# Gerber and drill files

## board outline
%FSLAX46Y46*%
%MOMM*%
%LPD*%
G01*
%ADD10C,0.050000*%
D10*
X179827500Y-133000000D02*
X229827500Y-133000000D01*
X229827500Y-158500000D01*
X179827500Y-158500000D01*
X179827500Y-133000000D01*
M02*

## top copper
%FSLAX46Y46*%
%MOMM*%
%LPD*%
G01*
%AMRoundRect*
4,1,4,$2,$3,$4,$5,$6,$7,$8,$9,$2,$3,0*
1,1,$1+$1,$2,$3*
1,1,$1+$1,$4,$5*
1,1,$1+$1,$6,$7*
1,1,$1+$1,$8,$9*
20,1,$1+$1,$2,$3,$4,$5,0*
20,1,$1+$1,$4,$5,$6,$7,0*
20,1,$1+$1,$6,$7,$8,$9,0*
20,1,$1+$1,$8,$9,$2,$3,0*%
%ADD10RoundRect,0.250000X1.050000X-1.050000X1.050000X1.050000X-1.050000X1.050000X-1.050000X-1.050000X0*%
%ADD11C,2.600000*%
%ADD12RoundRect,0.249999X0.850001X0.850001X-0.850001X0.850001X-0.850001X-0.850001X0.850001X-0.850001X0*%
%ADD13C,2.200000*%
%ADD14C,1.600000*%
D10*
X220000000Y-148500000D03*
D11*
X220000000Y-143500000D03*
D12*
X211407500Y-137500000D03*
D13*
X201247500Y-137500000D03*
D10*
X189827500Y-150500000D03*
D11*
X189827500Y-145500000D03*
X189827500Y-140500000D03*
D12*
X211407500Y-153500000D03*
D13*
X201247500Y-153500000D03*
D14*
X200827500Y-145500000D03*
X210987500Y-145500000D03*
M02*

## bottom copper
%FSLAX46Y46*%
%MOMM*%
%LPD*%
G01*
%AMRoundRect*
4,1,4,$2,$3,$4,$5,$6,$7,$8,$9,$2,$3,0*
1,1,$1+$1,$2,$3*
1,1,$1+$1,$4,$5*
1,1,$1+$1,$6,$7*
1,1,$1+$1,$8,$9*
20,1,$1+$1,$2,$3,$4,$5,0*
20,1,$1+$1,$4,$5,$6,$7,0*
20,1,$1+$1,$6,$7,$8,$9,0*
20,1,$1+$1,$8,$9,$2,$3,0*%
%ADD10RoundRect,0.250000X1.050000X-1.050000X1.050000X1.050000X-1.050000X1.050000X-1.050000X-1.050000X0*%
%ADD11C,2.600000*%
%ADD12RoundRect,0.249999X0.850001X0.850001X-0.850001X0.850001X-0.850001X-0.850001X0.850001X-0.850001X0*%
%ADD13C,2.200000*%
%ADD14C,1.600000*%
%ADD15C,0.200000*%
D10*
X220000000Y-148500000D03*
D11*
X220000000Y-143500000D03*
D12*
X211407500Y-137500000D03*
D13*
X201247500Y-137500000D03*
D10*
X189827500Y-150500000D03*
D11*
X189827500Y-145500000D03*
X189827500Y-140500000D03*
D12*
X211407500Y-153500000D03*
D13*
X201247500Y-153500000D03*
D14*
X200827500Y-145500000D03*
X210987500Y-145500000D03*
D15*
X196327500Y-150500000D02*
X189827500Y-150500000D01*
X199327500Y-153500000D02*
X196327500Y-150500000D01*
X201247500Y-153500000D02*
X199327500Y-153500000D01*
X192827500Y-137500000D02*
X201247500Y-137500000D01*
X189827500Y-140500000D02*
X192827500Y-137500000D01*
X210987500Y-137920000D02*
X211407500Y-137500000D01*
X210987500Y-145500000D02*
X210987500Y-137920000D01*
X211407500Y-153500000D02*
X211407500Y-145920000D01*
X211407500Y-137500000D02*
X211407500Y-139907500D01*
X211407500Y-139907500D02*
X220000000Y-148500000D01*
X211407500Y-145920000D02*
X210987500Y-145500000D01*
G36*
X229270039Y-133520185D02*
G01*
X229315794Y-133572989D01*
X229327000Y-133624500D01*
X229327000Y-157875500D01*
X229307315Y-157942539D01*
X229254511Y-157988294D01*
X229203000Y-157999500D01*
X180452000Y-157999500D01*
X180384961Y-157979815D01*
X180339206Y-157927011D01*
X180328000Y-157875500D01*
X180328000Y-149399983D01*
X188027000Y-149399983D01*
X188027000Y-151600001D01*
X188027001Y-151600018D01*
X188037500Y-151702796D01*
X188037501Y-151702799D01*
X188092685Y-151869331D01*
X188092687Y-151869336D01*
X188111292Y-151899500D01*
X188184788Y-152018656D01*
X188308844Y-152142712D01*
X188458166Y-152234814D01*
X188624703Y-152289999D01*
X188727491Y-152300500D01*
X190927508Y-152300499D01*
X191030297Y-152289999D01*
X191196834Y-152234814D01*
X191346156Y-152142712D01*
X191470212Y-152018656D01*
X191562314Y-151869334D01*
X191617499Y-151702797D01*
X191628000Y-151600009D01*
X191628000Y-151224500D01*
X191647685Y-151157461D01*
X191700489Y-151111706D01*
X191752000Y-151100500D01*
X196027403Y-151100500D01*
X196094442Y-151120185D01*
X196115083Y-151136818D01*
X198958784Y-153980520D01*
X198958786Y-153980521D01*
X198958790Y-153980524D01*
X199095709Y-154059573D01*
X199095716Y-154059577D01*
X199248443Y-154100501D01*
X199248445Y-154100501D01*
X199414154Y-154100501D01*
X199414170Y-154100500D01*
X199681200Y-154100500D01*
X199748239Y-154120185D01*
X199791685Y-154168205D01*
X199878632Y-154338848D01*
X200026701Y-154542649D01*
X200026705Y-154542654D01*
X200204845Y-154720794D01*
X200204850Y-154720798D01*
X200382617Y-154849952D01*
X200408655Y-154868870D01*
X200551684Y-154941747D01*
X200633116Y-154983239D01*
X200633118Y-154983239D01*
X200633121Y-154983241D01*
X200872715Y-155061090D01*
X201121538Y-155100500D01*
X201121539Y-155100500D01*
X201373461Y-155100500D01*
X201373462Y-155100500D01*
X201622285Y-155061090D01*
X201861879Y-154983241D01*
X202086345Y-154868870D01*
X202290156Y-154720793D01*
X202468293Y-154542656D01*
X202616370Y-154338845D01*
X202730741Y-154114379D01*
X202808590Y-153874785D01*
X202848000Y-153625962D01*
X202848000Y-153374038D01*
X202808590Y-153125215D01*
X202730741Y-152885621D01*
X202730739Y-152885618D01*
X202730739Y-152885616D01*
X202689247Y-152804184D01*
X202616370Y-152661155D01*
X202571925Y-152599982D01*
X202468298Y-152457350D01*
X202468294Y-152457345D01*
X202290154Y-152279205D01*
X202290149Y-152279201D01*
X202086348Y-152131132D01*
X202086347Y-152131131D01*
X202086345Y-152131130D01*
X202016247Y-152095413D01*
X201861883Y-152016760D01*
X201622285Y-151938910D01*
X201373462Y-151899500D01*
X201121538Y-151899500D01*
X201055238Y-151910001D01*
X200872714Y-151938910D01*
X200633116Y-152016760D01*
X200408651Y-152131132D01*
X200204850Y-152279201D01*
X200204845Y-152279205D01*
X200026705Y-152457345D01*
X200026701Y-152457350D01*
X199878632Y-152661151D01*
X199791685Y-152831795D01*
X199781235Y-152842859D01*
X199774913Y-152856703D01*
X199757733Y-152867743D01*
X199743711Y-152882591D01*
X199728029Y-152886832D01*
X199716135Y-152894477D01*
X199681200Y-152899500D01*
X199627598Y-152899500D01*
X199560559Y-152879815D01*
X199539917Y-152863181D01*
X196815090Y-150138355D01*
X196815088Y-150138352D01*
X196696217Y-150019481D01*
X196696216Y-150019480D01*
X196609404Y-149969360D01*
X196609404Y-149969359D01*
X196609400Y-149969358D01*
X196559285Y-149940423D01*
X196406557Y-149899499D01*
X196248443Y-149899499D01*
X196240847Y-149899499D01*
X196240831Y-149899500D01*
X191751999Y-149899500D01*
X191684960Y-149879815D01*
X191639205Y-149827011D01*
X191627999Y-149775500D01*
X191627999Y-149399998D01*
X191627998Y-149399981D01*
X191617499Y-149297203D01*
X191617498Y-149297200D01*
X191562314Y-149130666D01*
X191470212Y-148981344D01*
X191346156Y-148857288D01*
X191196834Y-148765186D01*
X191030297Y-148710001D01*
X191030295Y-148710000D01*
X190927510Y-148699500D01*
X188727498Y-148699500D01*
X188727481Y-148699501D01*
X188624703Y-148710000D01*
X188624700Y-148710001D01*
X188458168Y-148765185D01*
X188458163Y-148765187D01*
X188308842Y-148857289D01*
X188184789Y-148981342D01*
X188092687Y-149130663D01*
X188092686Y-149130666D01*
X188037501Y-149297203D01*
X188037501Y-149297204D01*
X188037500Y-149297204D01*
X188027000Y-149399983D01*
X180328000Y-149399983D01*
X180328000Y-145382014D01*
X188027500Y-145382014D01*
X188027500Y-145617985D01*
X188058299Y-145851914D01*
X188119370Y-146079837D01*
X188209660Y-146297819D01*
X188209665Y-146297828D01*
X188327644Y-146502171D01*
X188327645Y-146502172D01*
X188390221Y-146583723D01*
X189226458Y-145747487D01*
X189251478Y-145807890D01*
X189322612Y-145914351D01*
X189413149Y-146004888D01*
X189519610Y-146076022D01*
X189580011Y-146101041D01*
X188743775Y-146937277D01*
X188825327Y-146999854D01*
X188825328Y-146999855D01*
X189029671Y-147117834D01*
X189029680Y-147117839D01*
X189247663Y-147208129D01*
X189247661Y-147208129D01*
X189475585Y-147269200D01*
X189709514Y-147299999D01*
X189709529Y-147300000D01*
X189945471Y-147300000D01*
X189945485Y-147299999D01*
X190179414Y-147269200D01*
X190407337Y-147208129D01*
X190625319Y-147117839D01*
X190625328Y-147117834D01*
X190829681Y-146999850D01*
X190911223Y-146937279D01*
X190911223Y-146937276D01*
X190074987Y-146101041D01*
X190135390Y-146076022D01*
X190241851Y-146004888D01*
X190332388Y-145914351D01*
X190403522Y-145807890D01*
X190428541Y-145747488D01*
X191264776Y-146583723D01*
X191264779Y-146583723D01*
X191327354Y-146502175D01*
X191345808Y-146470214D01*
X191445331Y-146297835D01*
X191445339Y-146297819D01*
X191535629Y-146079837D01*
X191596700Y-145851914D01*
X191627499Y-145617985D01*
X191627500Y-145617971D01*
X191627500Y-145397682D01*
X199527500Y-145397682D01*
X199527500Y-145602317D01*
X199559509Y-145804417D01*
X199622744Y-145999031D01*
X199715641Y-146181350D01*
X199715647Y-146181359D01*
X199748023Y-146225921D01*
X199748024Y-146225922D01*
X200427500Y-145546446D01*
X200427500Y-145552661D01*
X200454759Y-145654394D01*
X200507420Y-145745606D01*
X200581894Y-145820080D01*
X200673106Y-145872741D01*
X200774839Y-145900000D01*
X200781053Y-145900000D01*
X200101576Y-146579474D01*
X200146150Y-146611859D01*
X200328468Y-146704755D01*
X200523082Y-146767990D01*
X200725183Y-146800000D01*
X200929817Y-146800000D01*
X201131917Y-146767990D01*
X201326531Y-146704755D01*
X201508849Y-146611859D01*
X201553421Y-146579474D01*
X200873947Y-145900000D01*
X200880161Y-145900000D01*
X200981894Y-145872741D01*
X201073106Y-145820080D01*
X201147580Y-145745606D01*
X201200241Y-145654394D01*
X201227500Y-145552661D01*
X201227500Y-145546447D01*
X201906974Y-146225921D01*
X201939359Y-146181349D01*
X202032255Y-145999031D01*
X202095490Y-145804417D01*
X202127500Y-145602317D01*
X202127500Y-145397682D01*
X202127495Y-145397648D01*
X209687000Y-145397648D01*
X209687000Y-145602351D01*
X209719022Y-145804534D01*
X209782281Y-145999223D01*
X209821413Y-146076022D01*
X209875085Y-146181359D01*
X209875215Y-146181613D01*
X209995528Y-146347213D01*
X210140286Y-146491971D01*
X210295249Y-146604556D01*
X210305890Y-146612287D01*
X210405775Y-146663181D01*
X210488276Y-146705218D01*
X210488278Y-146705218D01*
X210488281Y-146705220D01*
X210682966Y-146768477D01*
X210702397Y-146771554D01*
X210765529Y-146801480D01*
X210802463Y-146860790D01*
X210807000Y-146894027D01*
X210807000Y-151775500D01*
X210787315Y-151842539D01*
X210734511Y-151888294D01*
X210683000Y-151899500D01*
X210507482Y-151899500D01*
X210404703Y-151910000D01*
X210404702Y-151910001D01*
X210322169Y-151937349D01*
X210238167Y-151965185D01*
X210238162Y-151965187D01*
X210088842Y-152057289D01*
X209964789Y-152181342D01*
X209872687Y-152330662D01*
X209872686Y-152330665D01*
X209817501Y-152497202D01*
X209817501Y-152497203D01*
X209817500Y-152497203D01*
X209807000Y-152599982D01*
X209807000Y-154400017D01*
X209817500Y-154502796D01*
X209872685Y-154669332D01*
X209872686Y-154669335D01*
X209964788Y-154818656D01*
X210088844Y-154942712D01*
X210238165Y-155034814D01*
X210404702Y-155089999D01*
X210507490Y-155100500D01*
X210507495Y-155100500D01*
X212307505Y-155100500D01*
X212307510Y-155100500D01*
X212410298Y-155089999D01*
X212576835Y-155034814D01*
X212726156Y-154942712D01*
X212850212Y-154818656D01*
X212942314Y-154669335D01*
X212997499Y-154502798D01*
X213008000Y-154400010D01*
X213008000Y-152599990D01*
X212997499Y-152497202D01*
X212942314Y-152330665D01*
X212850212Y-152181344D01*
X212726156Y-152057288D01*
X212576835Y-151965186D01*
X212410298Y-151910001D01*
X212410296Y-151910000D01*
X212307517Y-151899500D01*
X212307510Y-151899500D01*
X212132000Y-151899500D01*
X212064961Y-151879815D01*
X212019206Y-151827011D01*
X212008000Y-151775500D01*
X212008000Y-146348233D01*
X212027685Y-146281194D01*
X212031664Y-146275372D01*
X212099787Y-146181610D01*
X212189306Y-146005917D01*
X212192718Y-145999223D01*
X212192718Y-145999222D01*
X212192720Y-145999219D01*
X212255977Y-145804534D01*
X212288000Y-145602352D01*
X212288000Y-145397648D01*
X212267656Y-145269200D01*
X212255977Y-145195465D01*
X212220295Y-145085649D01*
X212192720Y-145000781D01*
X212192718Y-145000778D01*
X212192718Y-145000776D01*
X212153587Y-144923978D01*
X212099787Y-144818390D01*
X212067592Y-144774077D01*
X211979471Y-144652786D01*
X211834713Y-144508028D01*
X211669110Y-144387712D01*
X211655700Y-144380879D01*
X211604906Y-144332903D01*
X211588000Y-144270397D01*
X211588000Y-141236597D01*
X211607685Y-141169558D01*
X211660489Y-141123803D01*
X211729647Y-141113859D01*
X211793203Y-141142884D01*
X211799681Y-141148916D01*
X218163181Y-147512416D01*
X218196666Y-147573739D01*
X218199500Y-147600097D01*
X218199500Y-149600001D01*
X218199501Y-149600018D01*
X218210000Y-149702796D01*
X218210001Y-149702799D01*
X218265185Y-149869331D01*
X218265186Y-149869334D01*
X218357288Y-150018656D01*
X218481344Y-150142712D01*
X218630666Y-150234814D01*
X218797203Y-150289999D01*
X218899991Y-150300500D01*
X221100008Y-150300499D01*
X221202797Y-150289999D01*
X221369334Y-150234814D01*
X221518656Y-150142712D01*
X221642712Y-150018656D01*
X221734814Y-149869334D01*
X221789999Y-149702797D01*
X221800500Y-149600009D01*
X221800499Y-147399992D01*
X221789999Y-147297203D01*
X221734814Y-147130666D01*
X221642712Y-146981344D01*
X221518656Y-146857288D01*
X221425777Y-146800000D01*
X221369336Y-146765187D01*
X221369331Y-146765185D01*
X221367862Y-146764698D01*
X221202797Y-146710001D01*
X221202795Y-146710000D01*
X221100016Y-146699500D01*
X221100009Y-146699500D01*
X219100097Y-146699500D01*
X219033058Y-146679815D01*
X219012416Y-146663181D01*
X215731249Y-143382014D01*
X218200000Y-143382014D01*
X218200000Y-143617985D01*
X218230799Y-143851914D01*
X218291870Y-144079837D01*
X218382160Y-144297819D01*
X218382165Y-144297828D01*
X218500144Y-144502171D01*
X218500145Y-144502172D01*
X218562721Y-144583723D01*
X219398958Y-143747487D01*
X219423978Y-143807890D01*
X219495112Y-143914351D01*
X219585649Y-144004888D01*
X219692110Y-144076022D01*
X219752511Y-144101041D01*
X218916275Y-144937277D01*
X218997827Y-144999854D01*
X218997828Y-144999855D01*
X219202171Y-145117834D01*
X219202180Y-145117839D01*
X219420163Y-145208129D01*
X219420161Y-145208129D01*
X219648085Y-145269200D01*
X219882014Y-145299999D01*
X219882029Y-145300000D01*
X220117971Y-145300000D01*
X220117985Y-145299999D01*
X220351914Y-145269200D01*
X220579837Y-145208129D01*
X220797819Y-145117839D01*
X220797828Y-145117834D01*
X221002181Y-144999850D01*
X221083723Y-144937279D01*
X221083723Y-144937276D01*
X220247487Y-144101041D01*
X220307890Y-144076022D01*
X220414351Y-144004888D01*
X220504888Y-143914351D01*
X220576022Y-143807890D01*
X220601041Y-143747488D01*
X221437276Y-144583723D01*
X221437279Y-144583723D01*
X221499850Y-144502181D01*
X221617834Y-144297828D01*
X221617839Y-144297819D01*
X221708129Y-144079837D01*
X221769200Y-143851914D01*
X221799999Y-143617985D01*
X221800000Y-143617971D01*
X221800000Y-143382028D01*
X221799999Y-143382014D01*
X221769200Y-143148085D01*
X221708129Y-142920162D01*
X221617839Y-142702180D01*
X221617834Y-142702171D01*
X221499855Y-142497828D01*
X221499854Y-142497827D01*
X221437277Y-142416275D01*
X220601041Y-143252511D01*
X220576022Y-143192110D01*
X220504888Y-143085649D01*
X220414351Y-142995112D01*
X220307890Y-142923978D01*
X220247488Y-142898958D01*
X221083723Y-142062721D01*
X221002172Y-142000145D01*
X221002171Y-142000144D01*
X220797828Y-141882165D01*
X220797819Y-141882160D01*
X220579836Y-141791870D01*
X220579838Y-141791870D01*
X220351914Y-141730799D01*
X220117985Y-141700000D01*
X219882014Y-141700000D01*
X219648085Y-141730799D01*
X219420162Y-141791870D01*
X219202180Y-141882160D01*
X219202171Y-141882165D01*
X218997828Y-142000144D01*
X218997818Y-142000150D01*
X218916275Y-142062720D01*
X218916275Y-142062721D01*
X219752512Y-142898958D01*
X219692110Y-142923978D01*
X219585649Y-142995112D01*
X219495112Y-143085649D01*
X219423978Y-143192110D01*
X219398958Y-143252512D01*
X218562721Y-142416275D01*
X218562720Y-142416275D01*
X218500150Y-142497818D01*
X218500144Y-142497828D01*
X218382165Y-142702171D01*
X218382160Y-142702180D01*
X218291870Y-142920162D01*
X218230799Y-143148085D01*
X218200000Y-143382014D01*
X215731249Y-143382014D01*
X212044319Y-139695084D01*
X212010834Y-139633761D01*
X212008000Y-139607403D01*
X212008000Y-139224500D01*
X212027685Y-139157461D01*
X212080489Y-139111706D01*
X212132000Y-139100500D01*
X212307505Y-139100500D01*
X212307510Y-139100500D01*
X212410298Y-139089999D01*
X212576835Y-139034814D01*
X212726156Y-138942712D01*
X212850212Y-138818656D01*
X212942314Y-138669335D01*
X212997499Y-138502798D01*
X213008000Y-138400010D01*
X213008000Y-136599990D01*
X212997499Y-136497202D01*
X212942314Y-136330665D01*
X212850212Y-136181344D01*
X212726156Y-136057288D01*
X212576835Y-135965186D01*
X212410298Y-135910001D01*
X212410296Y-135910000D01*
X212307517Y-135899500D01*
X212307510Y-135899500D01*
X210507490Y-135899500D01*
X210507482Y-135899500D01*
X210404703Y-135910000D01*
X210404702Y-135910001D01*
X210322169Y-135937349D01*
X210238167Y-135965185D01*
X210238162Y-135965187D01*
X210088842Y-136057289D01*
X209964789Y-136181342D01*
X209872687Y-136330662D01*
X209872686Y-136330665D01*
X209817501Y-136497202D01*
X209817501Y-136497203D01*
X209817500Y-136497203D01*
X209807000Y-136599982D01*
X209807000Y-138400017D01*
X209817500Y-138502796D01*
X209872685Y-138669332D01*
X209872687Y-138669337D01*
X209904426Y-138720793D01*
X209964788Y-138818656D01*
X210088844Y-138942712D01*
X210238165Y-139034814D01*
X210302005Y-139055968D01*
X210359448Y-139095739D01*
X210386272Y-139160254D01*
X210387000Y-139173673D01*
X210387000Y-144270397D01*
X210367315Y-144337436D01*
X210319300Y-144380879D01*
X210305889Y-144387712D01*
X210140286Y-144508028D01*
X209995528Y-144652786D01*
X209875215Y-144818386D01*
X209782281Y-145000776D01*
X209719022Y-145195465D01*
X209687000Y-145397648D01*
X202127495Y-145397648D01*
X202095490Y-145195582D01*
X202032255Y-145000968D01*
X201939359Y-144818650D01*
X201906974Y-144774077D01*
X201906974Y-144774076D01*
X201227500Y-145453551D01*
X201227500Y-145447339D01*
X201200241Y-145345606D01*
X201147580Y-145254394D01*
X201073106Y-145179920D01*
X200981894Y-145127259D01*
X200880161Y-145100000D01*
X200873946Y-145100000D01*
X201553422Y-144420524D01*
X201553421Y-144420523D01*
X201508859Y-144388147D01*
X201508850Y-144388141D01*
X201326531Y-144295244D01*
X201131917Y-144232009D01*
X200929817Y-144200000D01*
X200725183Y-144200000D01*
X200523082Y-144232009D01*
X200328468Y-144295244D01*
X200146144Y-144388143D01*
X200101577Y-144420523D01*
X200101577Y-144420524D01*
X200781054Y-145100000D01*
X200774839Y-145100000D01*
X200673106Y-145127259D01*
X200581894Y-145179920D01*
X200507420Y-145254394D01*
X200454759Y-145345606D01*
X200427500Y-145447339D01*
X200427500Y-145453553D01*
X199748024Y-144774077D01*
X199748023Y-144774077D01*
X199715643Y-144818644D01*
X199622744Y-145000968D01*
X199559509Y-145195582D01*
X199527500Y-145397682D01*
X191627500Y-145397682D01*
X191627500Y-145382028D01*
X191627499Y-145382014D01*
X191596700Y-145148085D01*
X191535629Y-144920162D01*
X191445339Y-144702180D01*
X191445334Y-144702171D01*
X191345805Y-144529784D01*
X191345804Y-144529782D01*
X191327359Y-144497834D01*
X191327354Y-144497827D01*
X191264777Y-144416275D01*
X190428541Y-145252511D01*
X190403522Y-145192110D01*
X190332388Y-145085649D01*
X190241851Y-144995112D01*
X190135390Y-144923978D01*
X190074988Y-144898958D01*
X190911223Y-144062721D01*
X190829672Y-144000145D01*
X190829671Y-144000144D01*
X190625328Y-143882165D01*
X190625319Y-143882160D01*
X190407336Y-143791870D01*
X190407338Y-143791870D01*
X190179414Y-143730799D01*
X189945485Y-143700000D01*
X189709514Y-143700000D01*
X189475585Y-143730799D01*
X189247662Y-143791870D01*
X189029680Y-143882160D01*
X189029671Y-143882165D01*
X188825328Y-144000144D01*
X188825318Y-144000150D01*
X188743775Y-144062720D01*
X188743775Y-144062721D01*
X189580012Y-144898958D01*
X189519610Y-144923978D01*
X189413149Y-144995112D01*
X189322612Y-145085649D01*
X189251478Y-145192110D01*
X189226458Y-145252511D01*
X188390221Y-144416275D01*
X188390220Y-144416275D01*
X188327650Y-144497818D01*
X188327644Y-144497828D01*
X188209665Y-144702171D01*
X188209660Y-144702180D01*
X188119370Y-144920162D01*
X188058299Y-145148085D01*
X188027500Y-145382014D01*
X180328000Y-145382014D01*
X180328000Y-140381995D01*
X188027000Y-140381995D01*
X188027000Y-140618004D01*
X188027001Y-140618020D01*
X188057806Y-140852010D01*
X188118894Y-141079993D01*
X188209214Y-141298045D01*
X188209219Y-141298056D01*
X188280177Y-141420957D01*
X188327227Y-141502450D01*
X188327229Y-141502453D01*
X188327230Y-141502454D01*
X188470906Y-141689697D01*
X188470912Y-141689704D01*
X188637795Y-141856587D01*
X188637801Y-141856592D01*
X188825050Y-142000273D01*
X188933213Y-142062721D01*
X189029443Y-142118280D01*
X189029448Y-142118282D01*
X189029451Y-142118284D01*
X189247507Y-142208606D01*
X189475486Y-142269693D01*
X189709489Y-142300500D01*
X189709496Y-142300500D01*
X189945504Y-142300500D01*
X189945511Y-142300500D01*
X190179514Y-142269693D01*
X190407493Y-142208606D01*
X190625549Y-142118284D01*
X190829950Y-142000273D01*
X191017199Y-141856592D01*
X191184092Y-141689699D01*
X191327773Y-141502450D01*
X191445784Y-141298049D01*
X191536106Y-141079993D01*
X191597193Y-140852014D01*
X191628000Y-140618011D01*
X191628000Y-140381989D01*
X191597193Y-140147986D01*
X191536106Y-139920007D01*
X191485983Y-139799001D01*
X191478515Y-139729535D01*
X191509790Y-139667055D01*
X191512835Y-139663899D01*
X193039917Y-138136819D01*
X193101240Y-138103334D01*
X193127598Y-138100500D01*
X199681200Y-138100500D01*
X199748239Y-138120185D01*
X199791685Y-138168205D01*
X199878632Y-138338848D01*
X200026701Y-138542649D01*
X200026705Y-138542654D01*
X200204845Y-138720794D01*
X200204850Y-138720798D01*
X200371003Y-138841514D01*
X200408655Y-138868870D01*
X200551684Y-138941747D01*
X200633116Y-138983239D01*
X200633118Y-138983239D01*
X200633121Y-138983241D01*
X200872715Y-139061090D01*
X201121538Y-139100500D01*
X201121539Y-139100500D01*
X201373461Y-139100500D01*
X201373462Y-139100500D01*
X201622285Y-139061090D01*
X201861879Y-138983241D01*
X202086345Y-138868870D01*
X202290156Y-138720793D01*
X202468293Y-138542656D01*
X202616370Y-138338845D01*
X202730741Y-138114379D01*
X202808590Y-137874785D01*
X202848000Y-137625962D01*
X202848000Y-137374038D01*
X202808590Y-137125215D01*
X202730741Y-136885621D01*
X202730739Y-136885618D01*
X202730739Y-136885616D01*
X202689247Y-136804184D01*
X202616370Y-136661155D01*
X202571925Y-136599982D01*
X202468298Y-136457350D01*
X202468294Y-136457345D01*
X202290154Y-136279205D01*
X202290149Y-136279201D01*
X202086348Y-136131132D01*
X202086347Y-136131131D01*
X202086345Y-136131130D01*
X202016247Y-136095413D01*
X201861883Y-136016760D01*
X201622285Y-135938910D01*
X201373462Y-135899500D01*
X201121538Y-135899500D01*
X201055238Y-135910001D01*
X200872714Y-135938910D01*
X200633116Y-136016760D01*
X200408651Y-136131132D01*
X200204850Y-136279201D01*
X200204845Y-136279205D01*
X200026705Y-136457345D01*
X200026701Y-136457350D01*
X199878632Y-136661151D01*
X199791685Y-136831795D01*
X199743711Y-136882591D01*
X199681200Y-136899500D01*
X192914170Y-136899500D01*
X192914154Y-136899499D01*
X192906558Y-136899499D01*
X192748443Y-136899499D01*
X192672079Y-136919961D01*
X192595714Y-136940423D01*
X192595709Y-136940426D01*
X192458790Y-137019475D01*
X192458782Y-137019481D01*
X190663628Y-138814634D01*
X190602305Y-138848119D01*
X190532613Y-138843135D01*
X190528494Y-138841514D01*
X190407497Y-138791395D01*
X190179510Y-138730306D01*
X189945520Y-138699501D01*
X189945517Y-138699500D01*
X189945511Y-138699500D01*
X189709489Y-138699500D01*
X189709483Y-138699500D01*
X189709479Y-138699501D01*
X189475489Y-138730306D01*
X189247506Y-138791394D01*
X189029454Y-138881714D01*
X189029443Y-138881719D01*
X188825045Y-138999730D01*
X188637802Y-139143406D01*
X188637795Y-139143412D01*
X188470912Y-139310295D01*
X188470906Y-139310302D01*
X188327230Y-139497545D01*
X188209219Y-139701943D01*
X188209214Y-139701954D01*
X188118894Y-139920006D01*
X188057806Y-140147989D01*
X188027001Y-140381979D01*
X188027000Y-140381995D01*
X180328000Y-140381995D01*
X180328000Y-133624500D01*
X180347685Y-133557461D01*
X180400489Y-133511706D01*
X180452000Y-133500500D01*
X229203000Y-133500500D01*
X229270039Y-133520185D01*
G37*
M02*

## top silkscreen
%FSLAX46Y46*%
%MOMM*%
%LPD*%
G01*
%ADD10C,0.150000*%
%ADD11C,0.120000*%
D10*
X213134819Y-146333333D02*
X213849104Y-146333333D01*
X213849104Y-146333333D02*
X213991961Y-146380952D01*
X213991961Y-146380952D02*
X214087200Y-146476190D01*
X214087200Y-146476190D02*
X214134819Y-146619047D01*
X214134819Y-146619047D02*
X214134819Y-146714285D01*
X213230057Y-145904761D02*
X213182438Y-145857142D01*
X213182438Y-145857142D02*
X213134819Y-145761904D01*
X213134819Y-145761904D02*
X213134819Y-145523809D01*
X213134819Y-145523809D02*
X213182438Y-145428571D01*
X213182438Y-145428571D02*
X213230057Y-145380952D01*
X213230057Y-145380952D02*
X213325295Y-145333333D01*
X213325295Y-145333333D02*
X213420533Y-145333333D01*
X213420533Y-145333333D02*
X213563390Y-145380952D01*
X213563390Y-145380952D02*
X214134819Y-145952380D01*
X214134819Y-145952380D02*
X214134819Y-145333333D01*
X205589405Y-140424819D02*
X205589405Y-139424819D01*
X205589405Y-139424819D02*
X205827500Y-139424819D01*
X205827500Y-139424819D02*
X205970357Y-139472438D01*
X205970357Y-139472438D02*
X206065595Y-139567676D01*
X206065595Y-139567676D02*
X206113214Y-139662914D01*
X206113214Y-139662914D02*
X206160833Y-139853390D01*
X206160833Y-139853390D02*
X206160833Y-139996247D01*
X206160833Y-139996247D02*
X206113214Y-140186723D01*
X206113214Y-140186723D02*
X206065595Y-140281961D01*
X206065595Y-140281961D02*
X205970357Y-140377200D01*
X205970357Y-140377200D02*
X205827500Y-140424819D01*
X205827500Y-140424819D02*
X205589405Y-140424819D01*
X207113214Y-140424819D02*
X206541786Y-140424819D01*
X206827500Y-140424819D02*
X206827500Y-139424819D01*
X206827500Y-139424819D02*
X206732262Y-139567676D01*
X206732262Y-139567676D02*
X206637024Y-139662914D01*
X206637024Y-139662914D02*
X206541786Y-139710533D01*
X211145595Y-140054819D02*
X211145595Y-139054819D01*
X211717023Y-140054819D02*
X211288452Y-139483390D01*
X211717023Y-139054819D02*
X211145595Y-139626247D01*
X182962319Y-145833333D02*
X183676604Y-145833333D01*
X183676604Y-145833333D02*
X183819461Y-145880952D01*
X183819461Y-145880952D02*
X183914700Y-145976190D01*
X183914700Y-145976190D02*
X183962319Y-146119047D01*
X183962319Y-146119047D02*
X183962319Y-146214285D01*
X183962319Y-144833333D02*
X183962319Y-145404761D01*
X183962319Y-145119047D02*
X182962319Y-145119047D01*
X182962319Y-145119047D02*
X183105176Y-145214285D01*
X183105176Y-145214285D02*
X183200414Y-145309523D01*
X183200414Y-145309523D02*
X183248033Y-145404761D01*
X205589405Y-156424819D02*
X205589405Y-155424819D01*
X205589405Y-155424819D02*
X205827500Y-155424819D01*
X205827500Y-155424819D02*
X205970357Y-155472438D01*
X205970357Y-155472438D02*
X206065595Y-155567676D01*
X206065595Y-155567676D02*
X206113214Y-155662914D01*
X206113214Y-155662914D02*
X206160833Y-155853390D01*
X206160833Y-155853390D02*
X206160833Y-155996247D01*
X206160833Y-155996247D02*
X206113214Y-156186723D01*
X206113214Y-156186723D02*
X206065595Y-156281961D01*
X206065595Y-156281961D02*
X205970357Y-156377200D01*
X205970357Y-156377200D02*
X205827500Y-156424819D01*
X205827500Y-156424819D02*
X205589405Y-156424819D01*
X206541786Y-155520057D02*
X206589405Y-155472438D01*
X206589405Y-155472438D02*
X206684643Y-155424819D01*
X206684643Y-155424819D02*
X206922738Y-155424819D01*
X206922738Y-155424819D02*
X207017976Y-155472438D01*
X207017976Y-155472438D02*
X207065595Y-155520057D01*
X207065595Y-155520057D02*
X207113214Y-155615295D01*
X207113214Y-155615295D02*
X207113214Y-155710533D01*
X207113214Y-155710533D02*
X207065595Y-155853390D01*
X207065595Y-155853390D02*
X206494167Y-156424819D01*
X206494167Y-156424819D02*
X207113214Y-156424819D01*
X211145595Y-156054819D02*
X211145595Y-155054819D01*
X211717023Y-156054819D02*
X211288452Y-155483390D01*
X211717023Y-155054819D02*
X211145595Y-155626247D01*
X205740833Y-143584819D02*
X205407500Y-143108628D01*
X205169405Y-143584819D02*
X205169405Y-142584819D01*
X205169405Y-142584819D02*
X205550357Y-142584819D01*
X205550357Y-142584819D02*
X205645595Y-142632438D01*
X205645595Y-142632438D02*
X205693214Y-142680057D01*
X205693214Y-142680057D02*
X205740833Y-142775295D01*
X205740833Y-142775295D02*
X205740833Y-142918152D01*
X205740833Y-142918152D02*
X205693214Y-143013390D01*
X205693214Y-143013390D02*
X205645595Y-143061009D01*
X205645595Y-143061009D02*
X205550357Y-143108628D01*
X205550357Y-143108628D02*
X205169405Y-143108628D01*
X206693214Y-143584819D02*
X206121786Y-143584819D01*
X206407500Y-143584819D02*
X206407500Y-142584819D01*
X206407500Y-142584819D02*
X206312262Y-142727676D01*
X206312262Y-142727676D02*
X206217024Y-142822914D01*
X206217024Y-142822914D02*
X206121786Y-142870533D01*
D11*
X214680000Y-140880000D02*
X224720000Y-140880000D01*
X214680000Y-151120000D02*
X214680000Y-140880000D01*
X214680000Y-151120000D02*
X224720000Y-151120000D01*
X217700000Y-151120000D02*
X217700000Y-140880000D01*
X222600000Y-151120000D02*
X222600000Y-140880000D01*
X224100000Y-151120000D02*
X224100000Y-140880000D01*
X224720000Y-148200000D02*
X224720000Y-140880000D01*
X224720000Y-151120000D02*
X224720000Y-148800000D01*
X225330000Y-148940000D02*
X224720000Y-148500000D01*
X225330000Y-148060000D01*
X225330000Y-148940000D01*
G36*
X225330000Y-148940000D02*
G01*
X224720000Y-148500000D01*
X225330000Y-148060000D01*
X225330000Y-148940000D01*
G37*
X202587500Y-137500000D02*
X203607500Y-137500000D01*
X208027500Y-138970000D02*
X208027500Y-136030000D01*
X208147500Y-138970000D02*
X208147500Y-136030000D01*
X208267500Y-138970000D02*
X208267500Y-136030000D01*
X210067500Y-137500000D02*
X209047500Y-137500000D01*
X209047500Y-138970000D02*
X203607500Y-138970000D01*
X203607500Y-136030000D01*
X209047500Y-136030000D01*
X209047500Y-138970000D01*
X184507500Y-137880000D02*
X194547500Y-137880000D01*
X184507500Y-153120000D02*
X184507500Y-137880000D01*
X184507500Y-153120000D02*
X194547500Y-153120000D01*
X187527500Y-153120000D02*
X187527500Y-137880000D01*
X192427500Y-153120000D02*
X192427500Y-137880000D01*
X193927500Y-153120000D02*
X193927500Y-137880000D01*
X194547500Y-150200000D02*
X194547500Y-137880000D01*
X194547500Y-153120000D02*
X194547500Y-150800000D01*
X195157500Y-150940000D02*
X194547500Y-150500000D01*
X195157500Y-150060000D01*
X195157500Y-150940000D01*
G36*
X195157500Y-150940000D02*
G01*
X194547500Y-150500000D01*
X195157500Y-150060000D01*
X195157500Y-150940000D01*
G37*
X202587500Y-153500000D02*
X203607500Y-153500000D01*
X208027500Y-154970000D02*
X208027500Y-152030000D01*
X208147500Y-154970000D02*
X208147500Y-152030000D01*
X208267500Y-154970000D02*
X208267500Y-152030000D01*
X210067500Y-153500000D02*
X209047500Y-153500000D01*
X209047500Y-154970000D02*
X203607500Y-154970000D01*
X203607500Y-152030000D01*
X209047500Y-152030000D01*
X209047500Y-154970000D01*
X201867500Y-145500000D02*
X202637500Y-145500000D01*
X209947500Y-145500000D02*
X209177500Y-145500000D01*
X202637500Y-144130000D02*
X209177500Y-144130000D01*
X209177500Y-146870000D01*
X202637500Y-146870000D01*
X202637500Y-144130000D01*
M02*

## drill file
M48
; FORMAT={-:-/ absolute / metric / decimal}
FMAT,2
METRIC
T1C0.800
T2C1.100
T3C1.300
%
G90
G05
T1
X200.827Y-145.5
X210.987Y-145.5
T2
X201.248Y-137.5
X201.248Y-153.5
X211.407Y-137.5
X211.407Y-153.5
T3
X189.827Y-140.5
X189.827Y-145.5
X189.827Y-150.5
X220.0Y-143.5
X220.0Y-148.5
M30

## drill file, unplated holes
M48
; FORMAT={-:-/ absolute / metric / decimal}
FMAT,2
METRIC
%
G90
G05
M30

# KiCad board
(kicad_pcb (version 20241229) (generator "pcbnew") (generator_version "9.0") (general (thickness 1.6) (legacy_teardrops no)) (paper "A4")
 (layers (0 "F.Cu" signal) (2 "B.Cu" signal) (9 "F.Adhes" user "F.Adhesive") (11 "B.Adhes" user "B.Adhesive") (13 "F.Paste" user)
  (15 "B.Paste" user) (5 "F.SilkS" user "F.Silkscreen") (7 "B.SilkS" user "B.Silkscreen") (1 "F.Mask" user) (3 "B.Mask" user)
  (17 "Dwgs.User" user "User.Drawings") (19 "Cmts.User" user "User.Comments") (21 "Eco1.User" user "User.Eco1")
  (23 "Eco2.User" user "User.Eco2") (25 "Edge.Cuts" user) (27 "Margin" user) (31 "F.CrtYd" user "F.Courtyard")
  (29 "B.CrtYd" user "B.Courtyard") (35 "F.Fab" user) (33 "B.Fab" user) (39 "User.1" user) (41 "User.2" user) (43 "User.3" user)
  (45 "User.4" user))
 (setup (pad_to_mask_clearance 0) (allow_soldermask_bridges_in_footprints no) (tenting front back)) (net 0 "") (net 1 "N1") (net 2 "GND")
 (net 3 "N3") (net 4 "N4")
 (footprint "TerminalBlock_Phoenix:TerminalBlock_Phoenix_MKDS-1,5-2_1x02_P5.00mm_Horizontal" (layer "F.Cu") (at 220 148.5 90)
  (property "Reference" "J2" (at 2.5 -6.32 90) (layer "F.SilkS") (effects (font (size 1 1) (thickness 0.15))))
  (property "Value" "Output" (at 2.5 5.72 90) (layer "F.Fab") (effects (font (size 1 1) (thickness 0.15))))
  (fp_line (start 7.62 -5.32) (end 7.62 4.72) (stroke (width 0.12) (type solid)) (layer "F.SilkS"))
  (fp_line (start -2.62 -5.32) (end 7.62 -5.32) (stroke (width 0.12) (type solid)) (layer "F.SilkS"))
  (fp_line (start -2.62 -5.32) (end -2.62 4.72) (stroke (width 0.12) (type solid)) (layer "F.SilkS"))
  (fp_line (start -2.62 -2.3) (end 7.62 -2.3) (stroke (width 0.12) (type solid)) (layer "F.SilkS"))
  (fp_line (start -2.62 2.6) (end 7.62 2.6) (stroke (width 0.12) (type solid)) (layer "F.SilkS"))
  (fp_line (start -2.62 4.1) (end 7.62 4.1) (stroke (width 0.12) (type solid)) (layer "F.SilkS"))
  (fp_line (start 0.3 4.72) (end 7.62 4.72) (stroke (width 0.12) (type solid)) (layer "F.SilkS"))
  (fp_line (start -2.62 4.72) (end -0.3 4.72) (stroke (width 0.12) (type solid)) (layer "F.SilkS"))
  (fp_poly (pts (xy 0 4.72) (xy 0.44 5.33) (xy -0.44 5.33)) (stroke (width 0.12) (type solid)) (fill yes) (layer "F.SilkS"))
  (pad "1" thru_hole roundrect (at 0 0 90) (size 2.6 2.6) (drill 1.3) (layers "*.Cu" "*.Mask") (remove_unused_layers no)
   (roundrect_rratio 0.096154) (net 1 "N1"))
  (pad "2" thru_hole circle (at 5 0 90) (size 2.6 2.6) (drill 1.3) (layers "*.Cu" "*.Mask") (remove_unused_layers no) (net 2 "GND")))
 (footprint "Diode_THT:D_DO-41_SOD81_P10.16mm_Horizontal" (layer "F.Cu") (at 211.4075 137.5 180)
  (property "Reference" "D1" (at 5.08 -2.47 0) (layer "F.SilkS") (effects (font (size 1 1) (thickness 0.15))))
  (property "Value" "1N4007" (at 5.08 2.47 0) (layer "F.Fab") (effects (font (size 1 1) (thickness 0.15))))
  (fp_line (start 8.82 0) (end 7.8 0) (stroke (width 0.12) (type solid)) (layer "F.SilkS"))
  (fp_line (start 3.38 -1.47) (end 3.38 1.47) (stroke (width 0.12) (type solid)) (layer "F.SilkS"))
  (fp_line (start 3.26 -1.47) (end 3.26 1.47) (stroke (width 0.12) (type solid)) (layer "F.SilkS"))
  (fp_line (start 3.14 -1.47) (end 3.14 1.47) (stroke (width 0.12) (type solid)) (layer "F.SilkS"))
  (fp_line (start 1.34 0) (end 2.36 0) (stroke (width 0.12) (type solid)) (layer "F.SilkS"))
  (fp_rect (start 2.36 -1.47) (end 7.8 1.47) (stroke (width 0.12) (type solid)) (fill no) (layer "F.SilkS"))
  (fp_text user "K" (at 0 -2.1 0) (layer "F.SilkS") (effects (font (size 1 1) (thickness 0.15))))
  (pad "1" thru_hole roundrect (at 0 0 180) (size 2.2 2.2) (drill 1.1) (layers "*.Cu" "*.Mask") (remove_unused_layers no)
   (roundrect_rratio 0.113636) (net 1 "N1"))
  (pad "2" thru_hole circle (at 10.16 0 180) (size 2.2 2.2) (drill 1.1) (layers "*.Cu" "*.Mask") (remove_unused_layers no) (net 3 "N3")))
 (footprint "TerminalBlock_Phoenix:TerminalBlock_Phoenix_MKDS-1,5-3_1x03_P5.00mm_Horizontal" (layer "F.Cu") (at 189.8275 150.5 90)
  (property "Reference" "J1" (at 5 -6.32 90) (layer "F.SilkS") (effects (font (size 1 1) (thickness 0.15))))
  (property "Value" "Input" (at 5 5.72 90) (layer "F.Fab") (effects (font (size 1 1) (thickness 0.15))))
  (fp_line (start 12.62 -5.32) (end 12.62 4.72) (stroke (width 0.12) (type solid)) (layer "F.SilkS"))
  (fp_line (start -2.62 -5.32) (end 12.62 -5.32) (stroke (width 0.12) (type solid)) (layer "F.SilkS"))
  (fp_line (start -2.62 -5.32) (end -2.62 4.72) (stroke (width 0.12) (type solid)) (layer "F.SilkS"))
  (fp_line (start -2.62 -2.3) (end 12.62 -2.3) (stroke (width 0.12) (type solid)) (layer "F.SilkS"))
  (fp_line (start -2.62 2.6) (end 12.62 2.6) (stroke (width 0.12) (type solid)) (layer "F.SilkS"))
  (fp_line (start -2.62 4.1) (end 12.62 4.1) (stroke (width 0.12) (type solid)) (layer "F.SilkS"))
  (fp_line (start 0.3 4.72) (end 12.62 4.72) (stroke (width 0.12) (type solid)) (layer "F.SilkS"))
  (fp_line (start -2.62 4.72) (end -0.3 4.72) (stroke (width 0.12) (type solid)) (layer "F.SilkS"))
  (fp_poly (pts (xy 0 4.72) (xy 0.44 5.33) (xy -0.44 5.33)) (stroke (width 0.12) (type solid)) (fill yes) (layer "F.SilkS"))
  (pad "1" thru_hole roundrect (at 0 0 90) (size 2.6 2.6) (drill 1.3) (layers "*.Cu" "*.Mask") (remove_unused_layers no)
   (roundrect_rratio 0.096154) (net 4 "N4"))
  (pad "2" thru_hole circle (at 5 0 90) (size 2.6 2.6) (drill 1.3) (layers "*.Cu" "*.Mask") (remove_unused_layers no) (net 2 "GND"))
  (pad "3" thru_hole circle (at 10 0 90) (size 2.6 2.6) (drill 1.3) (layers "*.Cu" "*.Mask") (remove_unused_layers no) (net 3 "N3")))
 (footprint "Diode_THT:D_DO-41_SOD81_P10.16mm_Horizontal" (layer "F.Cu") (at 211.4075 153.5 180)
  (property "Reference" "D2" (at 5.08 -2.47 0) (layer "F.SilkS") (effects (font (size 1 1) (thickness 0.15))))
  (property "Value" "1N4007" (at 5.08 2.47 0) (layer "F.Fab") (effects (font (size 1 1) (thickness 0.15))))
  (fp_line (start 8.82 0) (end 7.8 0) (stroke (width 0.12) (type solid)) (layer "F.SilkS"))
  (fp_line (start 3.38 -1.47) (end 3.38 1.47) (stroke (width 0.12) (type solid)) (layer "F.SilkS"))
  (fp_line (start 3.26 -1.47) (end 3.26 1.47) (stroke (width 0.12) (type solid)) (layer "F.SilkS"))
  (fp_line (start 3.14 -1.47) (end 3.14 1.47) (stroke (width 0.12) (type solid)) (layer "F.SilkS"))
  (fp_line (start 1.34 0) (end 2.36 0) (stroke (width 0.12) (type solid)) (layer "F.SilkS"))
  (fp_rect (start 2.36 -1.47) (end 7.8 1.47) (stroke (width 0.12) (type solid)) (fill no) (layer "F.SilkS"))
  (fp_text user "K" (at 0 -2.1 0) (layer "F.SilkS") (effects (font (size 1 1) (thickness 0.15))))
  (pad "1" thru_hole roundrect (at 0 0 180) (size 2.2 2.2) (drill 1.1) (layers "*.Cu" "*.Mask") (remove_unused_layers no)
   (roundrect_rratio 0.113636) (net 1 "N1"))
  (pad "2" thru_hole circle (at 10.16 0 180) (size 2.2 2.2) (drill 1.1) (layers "*.Cu" "*.Mask") (remove_unused_layers no) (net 4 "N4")))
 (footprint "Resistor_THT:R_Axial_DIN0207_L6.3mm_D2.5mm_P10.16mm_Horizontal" (layer "F.Cu") (at 200.8275 145.5)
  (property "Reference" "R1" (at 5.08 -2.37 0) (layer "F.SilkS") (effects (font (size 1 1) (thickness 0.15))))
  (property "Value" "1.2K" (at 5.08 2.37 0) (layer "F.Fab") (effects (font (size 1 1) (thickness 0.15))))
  (fp_line (start 1.04 0) (end 1.81 0) (stroke (width 0.12) (type solid)) (layer "F.SilkS"))
  (fp_line (start 9.12 0) (end 8.35 0) (stroke (width 0.12) (type solid)) (layer "F.SilkS"))
  (fp_rect (start 1.81 -1.37) (end 8.35 1.37) (stroke (width 0.12) (type solid)) (fill no) (layer "F.SilkS"))
  (pad "1" thru_hole circle (at 0 0) (size 1.6 1.6) (drill 0.8) (layers "*.Cu" "*.Mask") (remove_unused_layers no) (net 2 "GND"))
  (pad "2" thru_hole circle (at 10.16 0) (size 1.6 1.6) (drill 0.8) (layers "*.Cu" "*.Mask") (remove_unused_layers no) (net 1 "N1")))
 (gr_rect (start 179.8275 133) (end 229.8275 158.5) (stroke (width 0.05) (type default)) (fill no) (layer "Edge.Cuts"))
 (segment (start 196.3275 150.5) (end 189.8275 150.5) (width 0.2) (layer "B.Cu") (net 4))
 (segment (start 199.3275 153.5) (end 196.3275 150.5) (width 0.2) (layer "B.Cu") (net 4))
 (segment (start 201.2475 153.5) (end 199.3275 153.5) (width 0.2) (layer "B.Cu") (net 4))
 (segment (start 192.8275 137.5) (end 201.2475 137.5) (width 0.2) (layer "B.Cu") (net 3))
 (segment (start 189.8275 140.5) (end 192.8275 137.5) (width 0.2) (layer "B.Cu") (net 3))
 (segment (start 210.9875 137.92) (end 211.4075 137.5) (width 0.2) (layer "B.Cu") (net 1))
 (segment (start 210.9875 145.5) (end 210.9875 137.92) (width 0.2) (layer "B.Cu") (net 1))
 (segment (start 211.4075 153.5) (end 211.4075 145.92) (width 0.2) (layer "B.Cu") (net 1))
 (segment (start 211.4075 137.5) (end 211.4075 139.9075) (width 0.2) (layer "B.Cu") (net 1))
 (segment (start 211.4075 139.9075) (end 220 148.5) (width 0.2) (layer "B.Cu") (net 1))
 (segment (start 211.4075 145.92) (end 210.9875 145.5) (width 0.2) (layer "B.Cu") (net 1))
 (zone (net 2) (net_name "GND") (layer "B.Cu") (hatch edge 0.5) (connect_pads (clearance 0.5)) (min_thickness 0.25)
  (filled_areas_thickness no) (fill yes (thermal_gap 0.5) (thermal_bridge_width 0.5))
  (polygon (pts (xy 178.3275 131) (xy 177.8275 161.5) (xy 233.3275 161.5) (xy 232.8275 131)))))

